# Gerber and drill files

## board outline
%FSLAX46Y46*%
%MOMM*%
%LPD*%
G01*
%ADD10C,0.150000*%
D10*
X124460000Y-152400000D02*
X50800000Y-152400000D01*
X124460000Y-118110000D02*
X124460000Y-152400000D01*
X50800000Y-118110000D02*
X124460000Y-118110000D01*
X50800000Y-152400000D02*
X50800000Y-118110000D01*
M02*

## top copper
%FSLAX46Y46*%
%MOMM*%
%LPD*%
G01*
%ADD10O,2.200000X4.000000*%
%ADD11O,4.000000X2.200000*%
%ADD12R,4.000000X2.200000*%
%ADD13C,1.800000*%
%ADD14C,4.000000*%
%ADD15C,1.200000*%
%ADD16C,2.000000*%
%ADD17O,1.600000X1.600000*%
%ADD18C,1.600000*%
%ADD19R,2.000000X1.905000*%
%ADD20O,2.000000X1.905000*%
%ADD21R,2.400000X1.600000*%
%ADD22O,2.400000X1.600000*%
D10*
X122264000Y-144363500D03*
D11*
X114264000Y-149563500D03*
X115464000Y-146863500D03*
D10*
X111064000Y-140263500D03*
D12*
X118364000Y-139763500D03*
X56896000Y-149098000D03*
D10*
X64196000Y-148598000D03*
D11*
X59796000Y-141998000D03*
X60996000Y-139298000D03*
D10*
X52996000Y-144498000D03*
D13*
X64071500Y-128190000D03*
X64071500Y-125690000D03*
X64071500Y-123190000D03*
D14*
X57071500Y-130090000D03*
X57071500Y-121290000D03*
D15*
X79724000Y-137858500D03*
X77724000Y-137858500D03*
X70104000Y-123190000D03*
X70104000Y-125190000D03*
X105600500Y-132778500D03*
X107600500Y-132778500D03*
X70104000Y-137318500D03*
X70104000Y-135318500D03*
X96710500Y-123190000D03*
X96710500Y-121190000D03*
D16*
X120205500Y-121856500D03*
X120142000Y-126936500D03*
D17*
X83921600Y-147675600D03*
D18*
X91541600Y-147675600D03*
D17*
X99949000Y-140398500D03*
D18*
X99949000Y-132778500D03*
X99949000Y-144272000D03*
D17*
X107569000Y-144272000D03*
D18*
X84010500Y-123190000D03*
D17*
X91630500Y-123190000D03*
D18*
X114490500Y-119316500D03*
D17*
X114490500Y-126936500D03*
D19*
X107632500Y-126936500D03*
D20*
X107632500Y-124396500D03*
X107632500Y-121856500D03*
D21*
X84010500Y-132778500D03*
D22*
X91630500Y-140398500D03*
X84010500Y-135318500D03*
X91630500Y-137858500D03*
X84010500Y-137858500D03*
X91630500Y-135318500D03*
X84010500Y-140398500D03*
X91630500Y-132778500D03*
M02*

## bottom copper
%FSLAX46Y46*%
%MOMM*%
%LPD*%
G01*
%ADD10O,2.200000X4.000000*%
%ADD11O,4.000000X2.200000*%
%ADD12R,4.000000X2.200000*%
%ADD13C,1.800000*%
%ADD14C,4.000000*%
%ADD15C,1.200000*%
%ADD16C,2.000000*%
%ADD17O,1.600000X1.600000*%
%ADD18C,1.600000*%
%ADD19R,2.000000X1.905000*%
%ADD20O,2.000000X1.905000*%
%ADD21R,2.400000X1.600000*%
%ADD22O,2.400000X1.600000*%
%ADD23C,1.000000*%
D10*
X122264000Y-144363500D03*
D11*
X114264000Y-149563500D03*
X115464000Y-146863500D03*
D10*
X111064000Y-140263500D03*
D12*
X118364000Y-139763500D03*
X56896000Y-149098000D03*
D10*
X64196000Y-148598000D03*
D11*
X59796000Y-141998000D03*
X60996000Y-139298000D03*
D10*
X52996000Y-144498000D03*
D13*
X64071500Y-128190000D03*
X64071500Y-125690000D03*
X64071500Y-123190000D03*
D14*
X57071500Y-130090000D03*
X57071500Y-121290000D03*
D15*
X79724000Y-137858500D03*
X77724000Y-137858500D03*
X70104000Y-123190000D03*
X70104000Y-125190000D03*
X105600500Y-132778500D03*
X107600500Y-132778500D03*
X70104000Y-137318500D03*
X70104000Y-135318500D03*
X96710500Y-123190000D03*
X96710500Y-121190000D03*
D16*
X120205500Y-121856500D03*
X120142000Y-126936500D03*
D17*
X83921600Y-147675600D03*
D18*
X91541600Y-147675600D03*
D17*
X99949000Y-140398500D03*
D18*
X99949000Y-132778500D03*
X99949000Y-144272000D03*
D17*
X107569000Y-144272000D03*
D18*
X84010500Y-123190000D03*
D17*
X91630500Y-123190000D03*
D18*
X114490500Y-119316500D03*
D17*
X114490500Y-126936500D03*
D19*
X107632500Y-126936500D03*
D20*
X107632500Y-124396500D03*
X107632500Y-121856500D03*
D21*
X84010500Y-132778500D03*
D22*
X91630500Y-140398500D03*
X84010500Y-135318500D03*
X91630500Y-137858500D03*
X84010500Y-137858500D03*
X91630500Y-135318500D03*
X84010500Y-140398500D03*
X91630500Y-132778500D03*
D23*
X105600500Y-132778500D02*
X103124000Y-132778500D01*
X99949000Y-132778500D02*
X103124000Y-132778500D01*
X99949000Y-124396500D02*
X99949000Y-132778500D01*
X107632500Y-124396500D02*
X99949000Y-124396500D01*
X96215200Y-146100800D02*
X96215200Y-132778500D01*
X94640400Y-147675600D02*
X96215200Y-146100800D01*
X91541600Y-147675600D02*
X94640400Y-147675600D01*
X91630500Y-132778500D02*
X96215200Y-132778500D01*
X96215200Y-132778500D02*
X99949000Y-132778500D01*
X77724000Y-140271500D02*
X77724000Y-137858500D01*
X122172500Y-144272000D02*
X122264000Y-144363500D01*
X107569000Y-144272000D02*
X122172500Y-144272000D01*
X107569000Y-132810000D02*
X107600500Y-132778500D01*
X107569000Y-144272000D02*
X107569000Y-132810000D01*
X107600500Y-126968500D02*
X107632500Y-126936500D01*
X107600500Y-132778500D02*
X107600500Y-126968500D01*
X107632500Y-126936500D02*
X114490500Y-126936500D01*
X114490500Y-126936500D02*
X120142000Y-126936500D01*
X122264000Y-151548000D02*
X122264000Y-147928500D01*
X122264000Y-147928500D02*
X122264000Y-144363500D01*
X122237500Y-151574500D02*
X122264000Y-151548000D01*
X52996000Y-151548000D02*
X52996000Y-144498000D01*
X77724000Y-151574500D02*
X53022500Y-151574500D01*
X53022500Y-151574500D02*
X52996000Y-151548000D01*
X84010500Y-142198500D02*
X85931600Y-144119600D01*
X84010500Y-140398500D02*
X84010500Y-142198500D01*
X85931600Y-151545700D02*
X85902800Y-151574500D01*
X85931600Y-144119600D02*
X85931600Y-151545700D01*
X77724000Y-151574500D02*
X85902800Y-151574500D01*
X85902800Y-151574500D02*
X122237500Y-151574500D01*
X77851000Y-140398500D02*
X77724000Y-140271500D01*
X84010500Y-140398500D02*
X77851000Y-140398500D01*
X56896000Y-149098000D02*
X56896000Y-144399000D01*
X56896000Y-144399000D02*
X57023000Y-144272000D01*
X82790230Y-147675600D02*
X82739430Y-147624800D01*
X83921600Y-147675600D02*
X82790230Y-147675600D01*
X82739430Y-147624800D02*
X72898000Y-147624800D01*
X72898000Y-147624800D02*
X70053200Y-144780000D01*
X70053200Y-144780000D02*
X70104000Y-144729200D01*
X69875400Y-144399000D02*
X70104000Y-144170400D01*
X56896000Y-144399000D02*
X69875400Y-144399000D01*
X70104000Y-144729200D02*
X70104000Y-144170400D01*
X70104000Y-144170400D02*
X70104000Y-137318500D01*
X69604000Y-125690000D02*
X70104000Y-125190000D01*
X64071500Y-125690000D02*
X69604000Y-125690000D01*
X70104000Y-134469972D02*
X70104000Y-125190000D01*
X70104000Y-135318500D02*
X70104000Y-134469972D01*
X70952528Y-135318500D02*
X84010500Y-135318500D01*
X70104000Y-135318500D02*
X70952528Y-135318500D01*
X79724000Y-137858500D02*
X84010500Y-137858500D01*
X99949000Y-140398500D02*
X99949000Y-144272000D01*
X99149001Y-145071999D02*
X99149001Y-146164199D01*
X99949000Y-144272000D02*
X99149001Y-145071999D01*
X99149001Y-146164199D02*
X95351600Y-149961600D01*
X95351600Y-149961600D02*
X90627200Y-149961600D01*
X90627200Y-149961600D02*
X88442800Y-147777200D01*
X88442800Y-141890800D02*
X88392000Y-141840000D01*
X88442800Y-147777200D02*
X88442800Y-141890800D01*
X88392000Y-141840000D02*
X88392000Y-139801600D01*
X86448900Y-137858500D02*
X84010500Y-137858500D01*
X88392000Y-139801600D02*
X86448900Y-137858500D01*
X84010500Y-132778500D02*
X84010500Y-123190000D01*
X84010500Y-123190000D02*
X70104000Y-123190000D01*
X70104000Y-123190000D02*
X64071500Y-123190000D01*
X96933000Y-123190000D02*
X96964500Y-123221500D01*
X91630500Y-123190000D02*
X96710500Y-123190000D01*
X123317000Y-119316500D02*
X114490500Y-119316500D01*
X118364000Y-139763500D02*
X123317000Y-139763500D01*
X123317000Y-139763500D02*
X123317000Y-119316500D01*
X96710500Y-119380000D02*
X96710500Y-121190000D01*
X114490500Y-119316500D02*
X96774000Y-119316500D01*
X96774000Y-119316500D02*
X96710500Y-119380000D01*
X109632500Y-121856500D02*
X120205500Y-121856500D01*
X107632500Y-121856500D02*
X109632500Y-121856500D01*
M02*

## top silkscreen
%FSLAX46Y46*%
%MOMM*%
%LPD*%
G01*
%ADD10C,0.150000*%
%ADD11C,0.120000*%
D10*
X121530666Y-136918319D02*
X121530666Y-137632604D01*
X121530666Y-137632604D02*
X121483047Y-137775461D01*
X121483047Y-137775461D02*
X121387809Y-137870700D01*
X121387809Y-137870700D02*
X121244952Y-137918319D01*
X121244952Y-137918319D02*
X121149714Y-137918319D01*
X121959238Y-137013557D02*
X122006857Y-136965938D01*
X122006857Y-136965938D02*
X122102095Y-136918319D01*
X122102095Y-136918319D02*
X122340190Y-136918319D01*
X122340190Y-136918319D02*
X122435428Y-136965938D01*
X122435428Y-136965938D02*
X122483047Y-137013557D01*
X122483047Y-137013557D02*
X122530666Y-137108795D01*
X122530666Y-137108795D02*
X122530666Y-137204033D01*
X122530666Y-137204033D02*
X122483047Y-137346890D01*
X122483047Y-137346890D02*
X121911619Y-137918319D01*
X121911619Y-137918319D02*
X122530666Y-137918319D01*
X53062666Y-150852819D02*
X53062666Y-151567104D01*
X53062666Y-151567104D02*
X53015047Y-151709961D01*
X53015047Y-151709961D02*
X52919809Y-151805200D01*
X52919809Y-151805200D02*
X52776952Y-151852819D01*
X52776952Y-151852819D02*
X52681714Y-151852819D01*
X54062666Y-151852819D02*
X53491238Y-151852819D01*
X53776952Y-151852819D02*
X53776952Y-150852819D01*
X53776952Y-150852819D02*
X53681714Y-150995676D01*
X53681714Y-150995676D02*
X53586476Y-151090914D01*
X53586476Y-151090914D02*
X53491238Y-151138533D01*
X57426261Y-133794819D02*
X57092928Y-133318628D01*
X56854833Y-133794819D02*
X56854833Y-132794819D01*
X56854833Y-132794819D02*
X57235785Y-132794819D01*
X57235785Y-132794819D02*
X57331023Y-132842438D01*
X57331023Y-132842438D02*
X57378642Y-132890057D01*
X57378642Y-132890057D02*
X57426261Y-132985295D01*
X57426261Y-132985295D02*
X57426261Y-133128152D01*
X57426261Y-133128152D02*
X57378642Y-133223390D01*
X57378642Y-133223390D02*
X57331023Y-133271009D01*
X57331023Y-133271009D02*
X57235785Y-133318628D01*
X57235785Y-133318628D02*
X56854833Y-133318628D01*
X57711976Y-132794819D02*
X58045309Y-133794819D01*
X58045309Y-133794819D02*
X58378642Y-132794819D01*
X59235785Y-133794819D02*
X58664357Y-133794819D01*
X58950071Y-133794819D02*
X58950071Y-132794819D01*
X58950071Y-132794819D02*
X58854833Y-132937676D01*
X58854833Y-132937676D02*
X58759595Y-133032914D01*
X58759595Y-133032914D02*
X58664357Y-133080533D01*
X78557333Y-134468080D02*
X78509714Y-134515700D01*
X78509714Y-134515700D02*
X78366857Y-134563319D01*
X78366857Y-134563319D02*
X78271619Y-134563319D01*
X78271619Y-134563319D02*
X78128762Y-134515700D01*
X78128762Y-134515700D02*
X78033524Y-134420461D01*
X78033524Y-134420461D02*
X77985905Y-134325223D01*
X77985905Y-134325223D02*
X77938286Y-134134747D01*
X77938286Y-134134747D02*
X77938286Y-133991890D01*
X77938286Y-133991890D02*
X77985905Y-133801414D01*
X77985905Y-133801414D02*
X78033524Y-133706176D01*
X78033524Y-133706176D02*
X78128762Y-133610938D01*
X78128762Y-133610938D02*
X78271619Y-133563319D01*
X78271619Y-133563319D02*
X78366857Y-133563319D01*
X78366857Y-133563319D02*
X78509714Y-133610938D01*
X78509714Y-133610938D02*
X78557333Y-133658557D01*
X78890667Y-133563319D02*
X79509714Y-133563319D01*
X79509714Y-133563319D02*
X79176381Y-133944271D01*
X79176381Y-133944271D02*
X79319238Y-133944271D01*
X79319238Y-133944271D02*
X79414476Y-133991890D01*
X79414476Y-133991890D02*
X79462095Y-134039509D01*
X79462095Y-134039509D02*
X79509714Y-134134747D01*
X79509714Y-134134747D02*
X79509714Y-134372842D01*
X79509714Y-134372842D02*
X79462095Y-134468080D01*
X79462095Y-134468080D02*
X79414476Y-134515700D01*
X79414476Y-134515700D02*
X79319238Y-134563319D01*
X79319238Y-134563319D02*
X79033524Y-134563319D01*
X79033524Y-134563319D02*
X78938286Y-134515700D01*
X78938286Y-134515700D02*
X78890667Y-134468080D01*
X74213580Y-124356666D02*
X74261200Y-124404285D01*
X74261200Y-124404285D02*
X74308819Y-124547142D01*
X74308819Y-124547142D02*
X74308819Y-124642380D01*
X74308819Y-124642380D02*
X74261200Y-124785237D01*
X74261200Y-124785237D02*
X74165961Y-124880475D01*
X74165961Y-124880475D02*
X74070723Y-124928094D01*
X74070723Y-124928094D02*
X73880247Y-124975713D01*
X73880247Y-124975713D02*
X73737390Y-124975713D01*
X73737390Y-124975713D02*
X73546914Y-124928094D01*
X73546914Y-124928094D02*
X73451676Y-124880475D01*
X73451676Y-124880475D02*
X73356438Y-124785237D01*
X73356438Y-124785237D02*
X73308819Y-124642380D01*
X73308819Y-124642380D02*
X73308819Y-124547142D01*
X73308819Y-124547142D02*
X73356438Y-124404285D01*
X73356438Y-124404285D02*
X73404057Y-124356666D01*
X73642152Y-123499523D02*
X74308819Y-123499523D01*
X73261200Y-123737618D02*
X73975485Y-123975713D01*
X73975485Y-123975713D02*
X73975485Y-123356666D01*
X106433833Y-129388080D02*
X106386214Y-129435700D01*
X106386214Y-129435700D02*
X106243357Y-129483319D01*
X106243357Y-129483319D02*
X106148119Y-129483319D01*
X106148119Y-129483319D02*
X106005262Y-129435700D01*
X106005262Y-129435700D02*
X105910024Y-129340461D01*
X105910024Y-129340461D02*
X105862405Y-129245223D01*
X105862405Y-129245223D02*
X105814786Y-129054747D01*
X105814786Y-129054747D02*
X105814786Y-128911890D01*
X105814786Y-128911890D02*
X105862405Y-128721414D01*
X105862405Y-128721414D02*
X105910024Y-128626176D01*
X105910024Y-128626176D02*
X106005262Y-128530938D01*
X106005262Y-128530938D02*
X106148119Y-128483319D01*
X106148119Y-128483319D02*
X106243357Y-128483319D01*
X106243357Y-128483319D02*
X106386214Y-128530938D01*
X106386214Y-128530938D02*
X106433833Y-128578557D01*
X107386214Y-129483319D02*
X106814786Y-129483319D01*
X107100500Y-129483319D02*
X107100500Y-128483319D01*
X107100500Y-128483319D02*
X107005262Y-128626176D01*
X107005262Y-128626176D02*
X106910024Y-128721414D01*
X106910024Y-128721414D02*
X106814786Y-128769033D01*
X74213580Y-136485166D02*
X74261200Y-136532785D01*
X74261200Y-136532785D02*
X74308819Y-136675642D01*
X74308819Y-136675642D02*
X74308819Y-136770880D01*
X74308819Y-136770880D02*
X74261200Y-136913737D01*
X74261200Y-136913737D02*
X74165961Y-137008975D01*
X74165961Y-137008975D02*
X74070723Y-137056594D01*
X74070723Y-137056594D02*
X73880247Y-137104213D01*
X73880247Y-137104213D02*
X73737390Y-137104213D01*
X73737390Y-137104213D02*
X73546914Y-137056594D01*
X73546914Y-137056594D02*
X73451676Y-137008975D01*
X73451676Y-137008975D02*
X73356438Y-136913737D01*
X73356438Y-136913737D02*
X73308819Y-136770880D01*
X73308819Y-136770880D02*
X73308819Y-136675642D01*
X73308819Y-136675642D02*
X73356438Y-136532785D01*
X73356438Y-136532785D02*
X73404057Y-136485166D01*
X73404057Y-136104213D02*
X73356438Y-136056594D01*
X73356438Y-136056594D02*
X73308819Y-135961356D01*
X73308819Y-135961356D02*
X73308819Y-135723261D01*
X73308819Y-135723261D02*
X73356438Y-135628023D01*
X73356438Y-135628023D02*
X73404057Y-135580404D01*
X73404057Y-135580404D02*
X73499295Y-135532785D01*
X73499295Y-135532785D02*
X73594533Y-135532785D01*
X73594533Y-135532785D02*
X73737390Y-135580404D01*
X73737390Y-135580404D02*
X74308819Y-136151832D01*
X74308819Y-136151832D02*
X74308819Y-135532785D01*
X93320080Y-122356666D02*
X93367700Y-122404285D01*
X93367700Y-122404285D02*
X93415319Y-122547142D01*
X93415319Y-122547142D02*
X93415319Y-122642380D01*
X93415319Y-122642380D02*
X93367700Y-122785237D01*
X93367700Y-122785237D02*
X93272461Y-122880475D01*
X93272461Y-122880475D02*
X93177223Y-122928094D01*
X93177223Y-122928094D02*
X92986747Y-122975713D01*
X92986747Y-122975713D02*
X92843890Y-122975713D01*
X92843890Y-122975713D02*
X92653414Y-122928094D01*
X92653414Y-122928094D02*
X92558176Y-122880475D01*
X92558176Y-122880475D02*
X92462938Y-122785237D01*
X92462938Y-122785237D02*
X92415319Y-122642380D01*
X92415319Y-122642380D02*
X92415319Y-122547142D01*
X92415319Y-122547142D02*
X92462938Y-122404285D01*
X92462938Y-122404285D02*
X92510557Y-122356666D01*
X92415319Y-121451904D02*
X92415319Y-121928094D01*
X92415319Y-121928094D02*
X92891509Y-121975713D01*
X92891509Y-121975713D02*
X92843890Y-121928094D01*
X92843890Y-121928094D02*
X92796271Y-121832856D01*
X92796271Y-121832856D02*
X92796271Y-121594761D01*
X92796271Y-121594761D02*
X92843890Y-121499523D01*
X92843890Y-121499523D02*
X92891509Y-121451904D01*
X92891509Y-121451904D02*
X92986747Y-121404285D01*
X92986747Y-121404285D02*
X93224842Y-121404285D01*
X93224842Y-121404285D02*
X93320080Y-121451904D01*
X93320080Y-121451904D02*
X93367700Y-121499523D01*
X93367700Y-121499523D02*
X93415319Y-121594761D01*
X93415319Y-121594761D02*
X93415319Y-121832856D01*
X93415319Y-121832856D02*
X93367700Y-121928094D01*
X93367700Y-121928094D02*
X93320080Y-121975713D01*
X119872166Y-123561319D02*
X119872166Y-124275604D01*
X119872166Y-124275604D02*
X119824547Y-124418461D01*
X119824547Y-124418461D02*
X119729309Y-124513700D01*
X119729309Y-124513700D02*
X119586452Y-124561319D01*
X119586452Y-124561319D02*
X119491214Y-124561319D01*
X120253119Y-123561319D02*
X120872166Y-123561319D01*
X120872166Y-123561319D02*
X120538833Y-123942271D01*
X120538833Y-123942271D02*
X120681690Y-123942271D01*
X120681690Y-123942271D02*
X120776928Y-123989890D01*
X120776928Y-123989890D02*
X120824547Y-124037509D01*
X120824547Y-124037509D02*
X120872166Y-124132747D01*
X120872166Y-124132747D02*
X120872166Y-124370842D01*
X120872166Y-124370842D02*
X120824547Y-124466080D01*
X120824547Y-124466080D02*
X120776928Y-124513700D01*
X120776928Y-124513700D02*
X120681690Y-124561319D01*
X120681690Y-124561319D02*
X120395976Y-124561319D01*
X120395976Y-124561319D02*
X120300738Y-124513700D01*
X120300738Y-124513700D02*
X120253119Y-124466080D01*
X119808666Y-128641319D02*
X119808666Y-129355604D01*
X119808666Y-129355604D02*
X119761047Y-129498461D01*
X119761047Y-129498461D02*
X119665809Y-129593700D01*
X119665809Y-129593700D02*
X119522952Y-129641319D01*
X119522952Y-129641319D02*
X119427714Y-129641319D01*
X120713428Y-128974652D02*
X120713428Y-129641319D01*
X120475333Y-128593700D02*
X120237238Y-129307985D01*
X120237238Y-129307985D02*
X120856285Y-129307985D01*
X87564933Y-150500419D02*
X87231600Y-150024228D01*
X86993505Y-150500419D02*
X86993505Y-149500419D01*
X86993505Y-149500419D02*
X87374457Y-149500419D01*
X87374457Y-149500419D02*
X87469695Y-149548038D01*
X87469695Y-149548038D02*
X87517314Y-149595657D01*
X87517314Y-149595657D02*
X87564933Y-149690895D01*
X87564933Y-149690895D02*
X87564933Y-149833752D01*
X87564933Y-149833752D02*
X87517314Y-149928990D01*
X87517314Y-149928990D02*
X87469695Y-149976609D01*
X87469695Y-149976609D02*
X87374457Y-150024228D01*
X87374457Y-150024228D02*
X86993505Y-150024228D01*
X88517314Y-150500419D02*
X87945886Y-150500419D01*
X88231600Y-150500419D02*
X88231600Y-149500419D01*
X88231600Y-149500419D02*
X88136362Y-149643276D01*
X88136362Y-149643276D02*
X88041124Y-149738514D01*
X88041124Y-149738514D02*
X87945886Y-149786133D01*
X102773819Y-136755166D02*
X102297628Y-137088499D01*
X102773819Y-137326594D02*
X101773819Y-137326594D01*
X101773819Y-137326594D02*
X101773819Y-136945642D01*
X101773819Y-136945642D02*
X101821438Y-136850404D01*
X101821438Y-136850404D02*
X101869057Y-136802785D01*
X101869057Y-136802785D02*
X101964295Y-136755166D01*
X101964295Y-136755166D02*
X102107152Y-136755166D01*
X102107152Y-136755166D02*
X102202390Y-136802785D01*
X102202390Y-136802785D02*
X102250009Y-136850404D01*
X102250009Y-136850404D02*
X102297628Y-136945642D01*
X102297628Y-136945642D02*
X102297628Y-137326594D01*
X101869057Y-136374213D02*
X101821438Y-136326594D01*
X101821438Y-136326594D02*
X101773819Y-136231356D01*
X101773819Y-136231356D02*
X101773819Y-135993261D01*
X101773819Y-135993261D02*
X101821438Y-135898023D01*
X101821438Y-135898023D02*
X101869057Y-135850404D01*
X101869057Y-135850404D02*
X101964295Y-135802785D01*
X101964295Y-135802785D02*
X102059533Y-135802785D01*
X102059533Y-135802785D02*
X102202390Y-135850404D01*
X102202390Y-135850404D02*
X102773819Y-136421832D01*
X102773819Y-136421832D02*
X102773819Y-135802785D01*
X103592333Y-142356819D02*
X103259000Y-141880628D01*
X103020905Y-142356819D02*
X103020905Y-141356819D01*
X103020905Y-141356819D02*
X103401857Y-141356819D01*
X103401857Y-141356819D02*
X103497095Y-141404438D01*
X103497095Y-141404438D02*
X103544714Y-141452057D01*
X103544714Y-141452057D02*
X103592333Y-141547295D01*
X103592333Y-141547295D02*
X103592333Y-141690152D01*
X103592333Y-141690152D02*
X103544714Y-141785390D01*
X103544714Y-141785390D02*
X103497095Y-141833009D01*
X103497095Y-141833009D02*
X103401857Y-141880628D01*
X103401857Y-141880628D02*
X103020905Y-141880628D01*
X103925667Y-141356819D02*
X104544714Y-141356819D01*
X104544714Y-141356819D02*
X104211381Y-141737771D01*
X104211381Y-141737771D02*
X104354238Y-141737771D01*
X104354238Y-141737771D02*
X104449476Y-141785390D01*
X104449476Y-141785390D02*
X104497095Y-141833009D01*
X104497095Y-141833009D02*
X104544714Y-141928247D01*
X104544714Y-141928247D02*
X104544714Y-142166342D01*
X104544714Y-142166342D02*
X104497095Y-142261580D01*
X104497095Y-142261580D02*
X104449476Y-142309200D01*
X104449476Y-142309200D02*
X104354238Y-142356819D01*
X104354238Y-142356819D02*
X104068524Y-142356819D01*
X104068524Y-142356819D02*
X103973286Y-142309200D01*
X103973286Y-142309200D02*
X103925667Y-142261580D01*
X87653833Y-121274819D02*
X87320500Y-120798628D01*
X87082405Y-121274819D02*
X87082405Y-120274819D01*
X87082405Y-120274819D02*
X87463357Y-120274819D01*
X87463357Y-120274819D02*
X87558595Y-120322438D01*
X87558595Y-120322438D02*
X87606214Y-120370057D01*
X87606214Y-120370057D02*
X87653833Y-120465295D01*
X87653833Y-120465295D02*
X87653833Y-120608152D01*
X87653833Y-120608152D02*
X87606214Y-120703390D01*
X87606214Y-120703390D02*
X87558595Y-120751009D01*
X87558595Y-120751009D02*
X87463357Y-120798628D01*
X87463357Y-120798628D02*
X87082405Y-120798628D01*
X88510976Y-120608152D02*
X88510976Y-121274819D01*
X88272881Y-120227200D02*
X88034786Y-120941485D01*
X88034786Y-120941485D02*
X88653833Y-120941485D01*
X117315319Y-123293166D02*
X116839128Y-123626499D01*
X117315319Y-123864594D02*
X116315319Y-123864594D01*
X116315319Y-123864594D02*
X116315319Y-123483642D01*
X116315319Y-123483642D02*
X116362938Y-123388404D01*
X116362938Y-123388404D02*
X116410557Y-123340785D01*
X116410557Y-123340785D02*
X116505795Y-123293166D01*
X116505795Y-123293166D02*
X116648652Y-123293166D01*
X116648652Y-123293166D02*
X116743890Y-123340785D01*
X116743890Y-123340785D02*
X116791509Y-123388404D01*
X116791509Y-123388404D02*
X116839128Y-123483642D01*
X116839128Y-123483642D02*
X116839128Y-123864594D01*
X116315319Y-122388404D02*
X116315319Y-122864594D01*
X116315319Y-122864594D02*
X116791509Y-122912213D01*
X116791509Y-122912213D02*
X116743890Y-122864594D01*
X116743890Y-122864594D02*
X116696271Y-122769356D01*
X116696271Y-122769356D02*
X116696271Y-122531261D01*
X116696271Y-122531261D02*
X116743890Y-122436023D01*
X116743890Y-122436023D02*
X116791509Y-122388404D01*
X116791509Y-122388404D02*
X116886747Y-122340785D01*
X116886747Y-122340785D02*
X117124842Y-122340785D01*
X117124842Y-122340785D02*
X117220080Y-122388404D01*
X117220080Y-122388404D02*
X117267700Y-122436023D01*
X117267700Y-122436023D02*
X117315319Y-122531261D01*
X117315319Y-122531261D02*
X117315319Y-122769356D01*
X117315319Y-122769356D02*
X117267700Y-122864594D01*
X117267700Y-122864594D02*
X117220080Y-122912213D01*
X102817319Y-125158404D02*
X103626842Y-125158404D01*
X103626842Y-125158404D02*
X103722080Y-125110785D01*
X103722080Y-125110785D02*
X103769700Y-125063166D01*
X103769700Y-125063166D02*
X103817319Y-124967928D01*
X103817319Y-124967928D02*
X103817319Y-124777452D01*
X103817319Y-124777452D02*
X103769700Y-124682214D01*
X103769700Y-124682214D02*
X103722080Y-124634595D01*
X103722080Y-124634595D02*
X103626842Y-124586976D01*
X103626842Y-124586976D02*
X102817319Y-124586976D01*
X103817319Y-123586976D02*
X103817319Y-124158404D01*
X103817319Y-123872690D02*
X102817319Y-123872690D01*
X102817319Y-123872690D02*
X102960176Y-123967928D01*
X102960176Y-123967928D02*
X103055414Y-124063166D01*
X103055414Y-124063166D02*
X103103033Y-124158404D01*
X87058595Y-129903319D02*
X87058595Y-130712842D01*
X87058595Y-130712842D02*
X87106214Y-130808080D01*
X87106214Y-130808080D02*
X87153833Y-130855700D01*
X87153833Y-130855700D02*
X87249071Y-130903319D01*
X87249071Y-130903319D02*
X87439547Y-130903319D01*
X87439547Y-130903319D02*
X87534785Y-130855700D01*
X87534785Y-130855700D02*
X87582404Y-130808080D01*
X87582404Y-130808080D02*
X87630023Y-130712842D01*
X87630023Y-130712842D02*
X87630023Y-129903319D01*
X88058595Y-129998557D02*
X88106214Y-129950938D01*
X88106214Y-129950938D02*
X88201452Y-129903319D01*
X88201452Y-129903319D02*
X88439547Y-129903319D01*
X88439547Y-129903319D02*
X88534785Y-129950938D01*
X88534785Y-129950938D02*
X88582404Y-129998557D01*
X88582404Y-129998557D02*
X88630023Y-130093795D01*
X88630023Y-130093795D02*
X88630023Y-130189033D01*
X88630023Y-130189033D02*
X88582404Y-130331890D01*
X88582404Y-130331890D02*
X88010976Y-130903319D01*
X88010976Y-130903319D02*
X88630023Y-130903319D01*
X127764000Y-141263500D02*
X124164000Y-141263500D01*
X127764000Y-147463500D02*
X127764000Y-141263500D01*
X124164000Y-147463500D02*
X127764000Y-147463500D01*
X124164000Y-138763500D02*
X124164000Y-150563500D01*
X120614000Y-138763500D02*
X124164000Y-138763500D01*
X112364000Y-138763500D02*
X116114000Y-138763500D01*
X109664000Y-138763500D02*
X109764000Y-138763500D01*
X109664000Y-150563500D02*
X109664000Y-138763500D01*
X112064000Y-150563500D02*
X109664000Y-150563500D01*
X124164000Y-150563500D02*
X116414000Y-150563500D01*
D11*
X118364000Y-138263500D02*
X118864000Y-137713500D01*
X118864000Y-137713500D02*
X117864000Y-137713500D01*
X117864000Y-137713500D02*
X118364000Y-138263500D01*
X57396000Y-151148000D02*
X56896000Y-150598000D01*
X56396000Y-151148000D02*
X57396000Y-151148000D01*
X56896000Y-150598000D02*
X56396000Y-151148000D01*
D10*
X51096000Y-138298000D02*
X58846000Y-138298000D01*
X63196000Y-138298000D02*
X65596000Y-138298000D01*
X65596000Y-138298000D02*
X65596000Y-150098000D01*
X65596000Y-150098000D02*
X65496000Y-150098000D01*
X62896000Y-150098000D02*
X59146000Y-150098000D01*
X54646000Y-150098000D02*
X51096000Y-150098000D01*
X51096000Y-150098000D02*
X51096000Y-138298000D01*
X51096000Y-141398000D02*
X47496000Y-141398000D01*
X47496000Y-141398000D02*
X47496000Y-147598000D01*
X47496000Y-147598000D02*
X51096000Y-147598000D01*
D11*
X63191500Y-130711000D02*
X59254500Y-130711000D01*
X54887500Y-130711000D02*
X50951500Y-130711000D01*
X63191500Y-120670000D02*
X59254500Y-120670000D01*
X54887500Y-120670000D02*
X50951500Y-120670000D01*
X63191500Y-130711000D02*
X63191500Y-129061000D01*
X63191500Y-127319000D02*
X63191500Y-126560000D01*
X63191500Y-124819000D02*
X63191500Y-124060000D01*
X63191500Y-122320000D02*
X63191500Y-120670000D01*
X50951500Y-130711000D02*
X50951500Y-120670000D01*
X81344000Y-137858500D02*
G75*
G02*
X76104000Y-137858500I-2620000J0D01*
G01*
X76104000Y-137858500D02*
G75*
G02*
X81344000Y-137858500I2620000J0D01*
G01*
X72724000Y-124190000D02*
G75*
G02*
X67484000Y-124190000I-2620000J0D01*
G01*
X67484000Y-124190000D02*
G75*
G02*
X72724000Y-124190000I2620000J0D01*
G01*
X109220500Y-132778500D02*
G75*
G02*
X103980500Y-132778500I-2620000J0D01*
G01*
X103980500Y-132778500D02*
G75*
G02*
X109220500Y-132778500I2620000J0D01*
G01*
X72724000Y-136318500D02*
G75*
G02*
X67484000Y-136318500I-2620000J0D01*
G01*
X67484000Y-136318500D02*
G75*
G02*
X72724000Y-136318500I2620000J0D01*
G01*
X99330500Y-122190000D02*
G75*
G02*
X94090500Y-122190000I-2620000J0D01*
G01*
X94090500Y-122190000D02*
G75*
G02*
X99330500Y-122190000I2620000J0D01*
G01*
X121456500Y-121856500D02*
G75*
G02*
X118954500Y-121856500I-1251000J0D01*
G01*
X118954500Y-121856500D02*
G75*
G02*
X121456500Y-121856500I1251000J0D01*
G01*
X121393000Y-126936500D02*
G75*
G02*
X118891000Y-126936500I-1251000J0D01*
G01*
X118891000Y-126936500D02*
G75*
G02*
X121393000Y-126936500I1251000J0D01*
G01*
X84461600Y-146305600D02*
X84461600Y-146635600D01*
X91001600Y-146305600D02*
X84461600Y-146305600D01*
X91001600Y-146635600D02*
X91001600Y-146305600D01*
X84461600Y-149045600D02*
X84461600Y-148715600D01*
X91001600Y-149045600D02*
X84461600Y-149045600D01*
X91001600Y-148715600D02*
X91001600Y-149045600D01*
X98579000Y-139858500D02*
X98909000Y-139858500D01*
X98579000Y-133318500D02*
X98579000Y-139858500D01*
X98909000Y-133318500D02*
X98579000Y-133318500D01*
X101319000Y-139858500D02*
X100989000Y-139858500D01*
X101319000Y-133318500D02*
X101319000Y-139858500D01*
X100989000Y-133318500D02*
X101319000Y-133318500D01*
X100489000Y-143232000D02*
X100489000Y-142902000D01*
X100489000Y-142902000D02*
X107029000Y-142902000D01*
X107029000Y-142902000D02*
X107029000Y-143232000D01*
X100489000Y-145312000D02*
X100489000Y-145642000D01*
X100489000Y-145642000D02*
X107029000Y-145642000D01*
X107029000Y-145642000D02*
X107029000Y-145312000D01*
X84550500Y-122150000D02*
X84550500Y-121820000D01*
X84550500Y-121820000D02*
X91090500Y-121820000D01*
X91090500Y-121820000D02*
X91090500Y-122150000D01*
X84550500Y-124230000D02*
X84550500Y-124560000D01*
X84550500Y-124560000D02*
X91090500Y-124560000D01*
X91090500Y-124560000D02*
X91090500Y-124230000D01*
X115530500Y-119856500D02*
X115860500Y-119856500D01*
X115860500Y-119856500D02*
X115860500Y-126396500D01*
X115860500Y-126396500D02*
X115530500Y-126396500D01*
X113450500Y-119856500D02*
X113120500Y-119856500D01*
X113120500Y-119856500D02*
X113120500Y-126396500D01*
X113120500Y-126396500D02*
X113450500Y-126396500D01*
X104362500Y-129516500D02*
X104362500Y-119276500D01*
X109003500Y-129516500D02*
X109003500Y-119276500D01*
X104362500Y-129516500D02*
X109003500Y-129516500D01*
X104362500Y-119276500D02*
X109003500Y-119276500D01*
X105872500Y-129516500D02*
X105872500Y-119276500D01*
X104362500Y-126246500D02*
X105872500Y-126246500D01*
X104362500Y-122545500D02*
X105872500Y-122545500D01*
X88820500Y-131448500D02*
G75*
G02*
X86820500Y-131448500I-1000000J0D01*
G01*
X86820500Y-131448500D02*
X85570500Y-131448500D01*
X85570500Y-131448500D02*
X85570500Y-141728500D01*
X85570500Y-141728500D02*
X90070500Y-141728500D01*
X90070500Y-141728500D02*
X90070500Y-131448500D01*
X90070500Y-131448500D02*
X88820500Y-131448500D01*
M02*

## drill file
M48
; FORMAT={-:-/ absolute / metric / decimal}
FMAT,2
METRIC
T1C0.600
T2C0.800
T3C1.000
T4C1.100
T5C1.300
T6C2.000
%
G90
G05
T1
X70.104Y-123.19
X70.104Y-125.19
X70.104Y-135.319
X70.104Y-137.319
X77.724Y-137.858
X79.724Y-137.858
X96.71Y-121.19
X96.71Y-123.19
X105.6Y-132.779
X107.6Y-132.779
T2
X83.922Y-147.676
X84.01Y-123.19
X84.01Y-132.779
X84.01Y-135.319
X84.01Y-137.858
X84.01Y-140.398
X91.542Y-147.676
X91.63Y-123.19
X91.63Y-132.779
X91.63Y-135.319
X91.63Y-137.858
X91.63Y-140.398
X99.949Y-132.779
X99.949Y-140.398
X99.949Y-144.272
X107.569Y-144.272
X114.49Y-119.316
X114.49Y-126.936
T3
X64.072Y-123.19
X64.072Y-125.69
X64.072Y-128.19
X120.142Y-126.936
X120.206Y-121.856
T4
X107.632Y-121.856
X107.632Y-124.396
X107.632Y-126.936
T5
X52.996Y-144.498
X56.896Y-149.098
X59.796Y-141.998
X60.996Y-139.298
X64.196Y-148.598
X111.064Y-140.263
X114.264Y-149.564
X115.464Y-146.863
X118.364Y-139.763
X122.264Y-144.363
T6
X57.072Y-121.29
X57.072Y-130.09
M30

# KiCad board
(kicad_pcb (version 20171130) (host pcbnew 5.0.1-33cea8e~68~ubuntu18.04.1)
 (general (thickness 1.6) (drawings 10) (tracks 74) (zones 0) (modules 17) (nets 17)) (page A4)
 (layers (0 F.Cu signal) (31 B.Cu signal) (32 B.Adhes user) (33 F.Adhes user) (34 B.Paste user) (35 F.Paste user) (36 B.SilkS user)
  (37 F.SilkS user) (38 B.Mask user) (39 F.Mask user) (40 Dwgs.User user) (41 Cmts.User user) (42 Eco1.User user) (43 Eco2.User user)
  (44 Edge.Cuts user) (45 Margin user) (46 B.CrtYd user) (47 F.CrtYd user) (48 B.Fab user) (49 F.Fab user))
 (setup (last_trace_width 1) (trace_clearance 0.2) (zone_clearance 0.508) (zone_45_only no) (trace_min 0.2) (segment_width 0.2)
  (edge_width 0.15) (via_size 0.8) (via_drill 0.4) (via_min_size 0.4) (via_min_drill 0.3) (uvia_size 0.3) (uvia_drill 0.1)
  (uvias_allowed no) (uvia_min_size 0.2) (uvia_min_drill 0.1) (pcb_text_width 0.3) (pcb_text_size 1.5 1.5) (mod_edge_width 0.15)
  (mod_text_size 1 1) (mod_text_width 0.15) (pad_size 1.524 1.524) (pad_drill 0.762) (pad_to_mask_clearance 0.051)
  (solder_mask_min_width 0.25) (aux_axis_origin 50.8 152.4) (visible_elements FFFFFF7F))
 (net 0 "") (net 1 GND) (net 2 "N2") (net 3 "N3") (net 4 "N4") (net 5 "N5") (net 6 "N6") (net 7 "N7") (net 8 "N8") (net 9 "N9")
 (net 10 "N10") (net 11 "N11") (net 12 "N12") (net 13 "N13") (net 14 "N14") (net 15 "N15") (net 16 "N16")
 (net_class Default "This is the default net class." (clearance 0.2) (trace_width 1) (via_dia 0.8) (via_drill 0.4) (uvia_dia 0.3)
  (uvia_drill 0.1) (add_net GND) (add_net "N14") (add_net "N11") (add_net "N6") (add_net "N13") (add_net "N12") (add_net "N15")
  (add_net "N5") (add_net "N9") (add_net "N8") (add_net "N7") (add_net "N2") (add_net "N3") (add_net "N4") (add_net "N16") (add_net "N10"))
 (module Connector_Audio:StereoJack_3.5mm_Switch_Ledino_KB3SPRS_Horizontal (layer F.Cu) (at 118.364 139.7635 180)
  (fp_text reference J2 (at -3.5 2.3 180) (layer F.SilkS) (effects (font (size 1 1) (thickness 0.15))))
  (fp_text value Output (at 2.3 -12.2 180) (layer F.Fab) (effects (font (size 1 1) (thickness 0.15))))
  (fp_line (start -9.4 -1.5) (end -5.8 -1.5) (layer F.SilkS) (width 0.15))
  (fp_line (start -9.4 -7.7) (end -9.4 -1.5) (layer F.SilkS) (width 0.15))
  (fp_line (start -5.8 -7.7) (end -9.4 -7.7) (layer F.SilkS) (width 0.15))
  (fp_line (start -5.8 1) (end -5.8 -10.8) (layer F.SilkS) (width 0.15))
  (fp_line (start -2.25 1) (end -5.8 1) (layer F.SilkS) (width 0.15))
  (fp_line (start 6 1) (end 2.25 1) (layer F.SilkS) (width 0.15))
  (fp_line (start 8.7 1) (end 8.6 1) (layer F.SilkS) (width 0.15))
  (fp_line (start 8.7 -10.8) (end 8.7 1) (layer F.SilkS) (width 0.15))
  (fp_line (start 6.3 -10.8) (end 8.7 -10.8) (layer F.SilkS) (width 0.15))
  (fp_line (start -5.8 -10.8) (end 1.95 -10.8) (layer F.SilkS) (width 0.15))
  (fp_line (start 0 1.5) (end -0.5 2.05) (layer F.SilkS) (width 0.12))
  (fp_line (start -0.5 2.05) (end 0.5 2.05) (layer F.SilkS) (width 0.12))
  (fp_line (start 0.5 2.05) (end 0 1.5) (layer F.SilkS) (width 0.12))
  (pad S thru_hole oval (at -3.9 -4.6 180) (size 2.2 4) (drill 1.3) (layers *.Cu *.Mask) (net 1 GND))
  (pad R thru_hole oval (at 4.1 -9.8 180) (size 4 2.2) (drill 1.3) (layers *.Cu *.Mask) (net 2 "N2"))
  (pad RN thru_hole oval (at 2.9 -7.1 180) (size 4 2.2) (drill 1.3) (layers *.Cu *.Mask) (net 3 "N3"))
  (pad TN thru_hole oval (at 7.3 -0.5 270) (size 4 2.2) (drill 1.3) (layers *.Cu *.Mask) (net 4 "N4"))
  (pad T thru_hole rect (at 0 0 180) (size 4 2.2) (drill 1.3) (layers *.Cu *.Mask) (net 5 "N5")))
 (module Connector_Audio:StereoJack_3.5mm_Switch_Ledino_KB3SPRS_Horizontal (layer F.Cu) (at 56.896 149.098)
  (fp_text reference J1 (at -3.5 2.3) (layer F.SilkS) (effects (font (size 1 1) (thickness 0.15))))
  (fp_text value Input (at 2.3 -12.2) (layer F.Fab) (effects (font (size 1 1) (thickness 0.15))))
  (fp_line (start 0.5 2.05) (end 0 1.5) (layer F.SilkS) (width 0.12))
  (fp_line (start -0.5 2.05) (end 0.5 2.05) (layer F.SilkS) (width 0.12))
  (fp_line (start 0 1.5) (end -0.5 2.05) (layer F.SilkS) (width 0.12))
  (fp_line (start -5.8 -10.8) (end 1.95 -10.8) (layer F.SilkS) (width 0.15))
  (fp_line (start 6.3 -10.8) (end 8.7 -10.8) (layer F.SilkS) (width 0.15))
  (fp_line (start 8.7 -10.8) (end 8.7 1) (layer F.SilkS) (width 0.15))
  (fp_line (start 8.7 1) (end 8.6 1) (layer F.SilkS) (width 0.15))
  (fp_line (start 6 1) (end 2.25 1) (layer F.SilkS) (width 0.15))
  (fp_line (start -2.25 1) (end -5.8 1) (layer F.SilkS) (width 0.15))
  (fp_line (start -5.8 1) (end -5.8 -10.8) (layer F.SilkS) (width 0.15))
  (fp_line (start -5.8 -7.7) (end -9.4 -7.7) (layer F.SilkS) (width 0.15))
  (fp_line (start -9.4 -7.7) (end -9.4 -1.5) (layer F.SilkS) (width 0.15))
  (fp_line (start -9.4 -1.5) (end -5.8 -1.5) (layer F.SilkS) (width 0.15))
  (pad T thru_hole rect (at 0 0) (size 4 2.2) (drill 1.3) (layers *.Cu *.Mask) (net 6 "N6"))
  (pad TN thru_hole oval (at 7.3 -0.5 90) (size 4 2.2) (drill 1.3) (layers *.Cu *.Mask) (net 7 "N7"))
  (pad RN thru_hole oval (at 2.9 -7.1) (size 4 2.2) (drill 1.3) (layers *.Cu *.Mask) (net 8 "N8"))
  (pad R thru_hole oval (at 4.1 -9.8) (size 4 2.2) (drill 1.3) (layers *.Cu *.Mask) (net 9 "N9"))
  (pad S thru_hole oval (at -3.9 -4.6) (size 2.2 4) (drill 1.3) (layers *.Cu *.Mask) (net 1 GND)))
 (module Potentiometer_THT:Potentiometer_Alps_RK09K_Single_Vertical (layer F.Cu) (at 64.0715 123.19 180)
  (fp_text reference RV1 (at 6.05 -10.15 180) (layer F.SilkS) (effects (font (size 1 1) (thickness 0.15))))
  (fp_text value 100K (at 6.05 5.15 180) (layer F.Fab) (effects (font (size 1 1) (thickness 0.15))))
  (fp_line (start 0.88 -7.521) (end 4.817 -7.521) (layer F.SilkS) (width 0.12))
  (fp_line (start 9.184 -7.521) (end 13.12 -7.521) (layer F.SilkS) (width 0.12))
  (fp_line (start 0.88 2.52) (end 4.817 2.52) (layer F.SilkS) (width 0.12))
  (fp_line (start 9.184 2.52) (end 13.12 2.52) (layer F.SilkS) (width 0.12))
  (fp_line (start 0.88 -7.521) (end 0.88 -5.871) (layer F.SilkS) (width 0.12))
  (fp_line (start 0.88 -4.129) (end 0.88 -3.37) (layer F.SilkS) (width 0.12))
  (fp_line (start 0.88 -1.629) (end 0.88 -0.87) (layer F.SilkS) (width 0.12))
  (fp_line (start 0.88 0.87) (end 0.88 2.52) (layer F.SilkS) (width 0.12))
  (fp_line (start 13.12 -7.521) (end 13.12 2.52) (layer F.SilkS) (width 0.12))
  (pad 3 thru_hole circle (at 0 -5 180) (size 1.8 1.8) (drill 1) (layers *.Cu *.Mask) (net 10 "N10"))
  (pad 2 thru_hole circle (at 0 -2.5 180) (size 1.8 1.8) (drill 1) (layers *.Cu *.Mask) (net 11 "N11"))
  (pad 1 thru_hole circle (at 0 0 180) (size 1.8 1.8) (drill 1) (layers *.Cu *.Mask) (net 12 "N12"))
  (pad "" np_thru_hole circle (at 7 -6.9 180) (size 4 4) (drill 2) (layers *.Cu *.Mask))
  (pad "" np_thru_hole circle (at 7 1.9 180) (size 4 4) (drill 2) (layers *.Cu *.Mask)))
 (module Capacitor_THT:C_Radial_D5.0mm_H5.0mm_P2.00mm (layer F.Cu) (at 77.724 137.8585)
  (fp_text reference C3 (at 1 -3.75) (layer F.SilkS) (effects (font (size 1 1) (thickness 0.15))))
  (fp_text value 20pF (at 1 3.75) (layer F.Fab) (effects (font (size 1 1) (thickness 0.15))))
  (fp_circle (center 1 0) (end 3.62 0) (layer F.SilkS) (width 0.12))
  (pad 2 thru_hole circle (at 2 0) (size 1.2 1.2) (drill 0.6) (layers *.Cu *.Mask) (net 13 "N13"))
  (pad 1 thru_hole circle (at 0 0) (size 1.2 1.2) (drill 0.6) (layers *.Cu *.Mask) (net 1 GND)))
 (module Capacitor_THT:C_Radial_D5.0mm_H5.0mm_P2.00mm (layer F.Cu) (at 70.104 123.19 270)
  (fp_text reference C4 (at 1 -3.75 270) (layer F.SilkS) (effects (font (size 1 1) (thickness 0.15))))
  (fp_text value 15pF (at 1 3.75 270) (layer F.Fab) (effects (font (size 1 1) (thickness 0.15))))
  (fp_circle (center 1 0) (end 3.62 0) (layer F.SilkS) (width 0.12))
  (pad 1 thru_hole circle (at 0 0 270) (size 1.2 1.2) (drill 0.6) (layers *.Cu *.Mask) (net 12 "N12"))
  (pad 2 thru_hole circle (at 2 0 270) (size 1.2 1.2) (drill 0.6) (layers *.Cu *.Mask) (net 11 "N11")))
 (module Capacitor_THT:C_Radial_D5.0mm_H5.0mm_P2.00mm (layer F.Cu) (at 105.6005 132.7785)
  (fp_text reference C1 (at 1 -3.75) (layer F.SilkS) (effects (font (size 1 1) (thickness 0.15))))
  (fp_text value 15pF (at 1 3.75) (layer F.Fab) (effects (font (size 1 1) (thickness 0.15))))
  (fp_circle (center 1 0) (end 3.62 0) (layer F.SilkS) (width 0.12))
  (pad 1 thru_hole circle (at 0 0) (size 1.2 1.2) (drill 0.6) (layers *.Cu *.Mask) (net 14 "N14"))
  (pad 2 thru_hole circle (at 2 0) (size 1.2 1.2) (drill 0.6) (layers *.Cu *.Mask) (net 1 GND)))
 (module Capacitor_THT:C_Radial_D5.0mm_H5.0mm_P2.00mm (layer F.Cu) (at 70.104 135.3185 270)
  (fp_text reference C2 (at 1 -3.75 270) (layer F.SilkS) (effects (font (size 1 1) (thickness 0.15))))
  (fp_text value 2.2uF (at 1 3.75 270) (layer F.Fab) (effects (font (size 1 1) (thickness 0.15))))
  (fp_circle (center 1 0) (end 3.62 0) (layer F.SilkS) (width 0.12))
  (pad 2 thru_hole circle (at 2 0 270) (size 1.2 1.2) (drill 0.6) (layers *.Cu *.Mask) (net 6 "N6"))
  (pad 1 thru_hole circle (at 0 0 270) (size 1.2 1.2) (drill 0.6) (layers *.Cu *.Mask) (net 11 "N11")))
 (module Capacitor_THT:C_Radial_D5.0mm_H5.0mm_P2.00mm (layer F.Cu) (at 96.7105 123.19 90)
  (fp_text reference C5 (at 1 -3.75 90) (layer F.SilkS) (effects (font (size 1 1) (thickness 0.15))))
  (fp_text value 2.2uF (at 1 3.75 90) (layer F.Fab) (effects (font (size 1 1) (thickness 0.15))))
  (fp_circle (center 1 0) (end 3.62 0) (layer F.SilkS) (width 0.12))
  (pad 1 thru_hole circle (at 0 0 90) (size 1.2 1.2) (drill 0.6) (layers *.Cu *.Mask) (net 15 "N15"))
  (pad 2 thru_hole circle (at 2 0 90) (size 1.2 1.2) (drill 0.6) (layers *.Cu *.Mask) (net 5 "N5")))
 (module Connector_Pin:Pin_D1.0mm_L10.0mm (layer F.Cu) (at 120.2055 121.8565)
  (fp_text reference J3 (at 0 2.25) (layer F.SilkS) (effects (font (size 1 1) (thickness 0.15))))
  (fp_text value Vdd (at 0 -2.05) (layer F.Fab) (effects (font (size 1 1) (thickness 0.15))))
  (fp_circle (center 0 0) (end 1.25 0.05) (layer F.SilkS) (width 0.12))
  (pad 1 thru_hole circle (at 0 0) (size 2 2) (drill 1) (layers *.Cu *.Mask) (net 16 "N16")))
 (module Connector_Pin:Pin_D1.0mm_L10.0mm (layer F.Cu) (at 120.142 126.9365)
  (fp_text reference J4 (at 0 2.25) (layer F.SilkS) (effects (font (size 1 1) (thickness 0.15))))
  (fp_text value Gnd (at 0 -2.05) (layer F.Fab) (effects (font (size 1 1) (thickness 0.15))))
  (fp_circle (center 0 0) (end 1.25 0.05) (layer F.SilkS) (width 0.12))
  (pad 1 thru_hole circle (at 0 0) (size 2 2) (drill 1) (layers *.Cu *.Mask) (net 1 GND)))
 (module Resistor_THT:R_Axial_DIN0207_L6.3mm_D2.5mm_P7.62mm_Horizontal (layer F.Cu) (at 91.5416 147.6756 180)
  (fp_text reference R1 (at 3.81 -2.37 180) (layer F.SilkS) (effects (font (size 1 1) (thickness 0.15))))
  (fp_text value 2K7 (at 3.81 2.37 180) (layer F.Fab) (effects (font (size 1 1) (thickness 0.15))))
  (fp_line (start 7.08 1.37) (end 7.08 1.04) (layer F.SilkS) (width 0.12))
  (fp_line (start 0.54 1.37) (end 7.08 1.37) (layer F.SilkS) (width 0.12))
  (fp_line (start 0.54 1.04) (end 0.54 1.37) (layer F.SilkS) (width 0.12))
  (fp_line (start 7.08 -1.37) (end 7.08 -1.04) (layer F.SilkS) (width 0.12))
  (fp_line (start 0.54 -1.37) (end 7.08 -1.37) (layer F.SilkS) (width 0.12))
  (fp_line (start 0.54 -1.04) (end 0.54 -1.37) (layer F.SilkS) (width 0.12))
  (pad 2 thru_hole oval (at 7.62 0 180) (size 1.6 1.6) (drill 0.8) (layers *.Cu *.Mask) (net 6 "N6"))
  (pad 1 thru_hole circle (at 0 0 180) (size 1.6 1.6) (drill 0.8) (layers *.Cu *.Mask) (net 14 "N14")))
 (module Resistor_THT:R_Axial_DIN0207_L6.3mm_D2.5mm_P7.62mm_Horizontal (layer F.Cu) (at 99.949 132.7785 270)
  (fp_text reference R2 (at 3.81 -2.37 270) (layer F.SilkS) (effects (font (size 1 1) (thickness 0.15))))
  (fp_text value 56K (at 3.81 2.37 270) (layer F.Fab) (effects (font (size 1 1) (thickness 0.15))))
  (fp_line (start 7.08 1.37) (end 7.08 1.04) (layer F.SilkS) (width 0.12))
  (fp_line (start 0.54 1.37) (end 7.08 1.37) (layer F.SilkS) (width 0.12))
  (fp_line (start 0.54 1.04) (end 0.54 1.37) (layer F.SilkS) (width 0.12))
  (fp_line (start 7.08 -1.37) (end 7.08 -1.04) (layer F.SilkS) (width 0.12))
  (fp_line (start 0.54 -1.37) (end 7.08 -1.37) (layer F.SilkS) (width 0.12))
  (fp_line (start 0.54 -1.04) (end 0.54 -1.37) (layer F.SilkS) (width 0.12))
  (pad 2 thru_hole oval (at 7.62 0 270) (size 1.6 1.6) (drill 0.8) (layers *.Cu *.Mask) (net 13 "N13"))
  (pad 1 thru_hole circle (at 0 0 270) (size 1.6 1.6) (drill 0.8) (layers *.Cu *.Mask) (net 14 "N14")))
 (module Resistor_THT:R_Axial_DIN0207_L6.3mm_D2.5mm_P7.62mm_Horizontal (layer F.Cu) (at 99.949 144.272)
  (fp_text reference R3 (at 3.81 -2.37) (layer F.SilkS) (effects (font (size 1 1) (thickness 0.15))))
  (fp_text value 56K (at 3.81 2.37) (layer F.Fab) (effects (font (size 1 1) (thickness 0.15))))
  (fp_line (start 0.54 -1.04) (end 0.54 -1.37) (layer F.SilkS) (width 0.12))
  (fp_line (start 0.54 -1.37) (end 7.08 -1.37) (layer F.SilkS) (width 0.12))
  (fp_line (start 7.08 -1.37) (end 7.08 -1.04) (layer F.SilkS) (width 0.12))
  (fp_line (start 0.54 1.04) (end 0.54 1.37) (layer F.SilkS) (width 0.12))
  (fp_line (start 0.54 1.37) (end 7.08 1.37) (layer F.SilkS) (width 0.12))
  (fp_line (start 7.08 1.37) (end 7.08 1.04) (layer F.SilkS) (width 0.12))
  (pad 1 thru_hole circle (at 0 0) (size 1.6 1.6) (drill 0.8) (layers *.Cu *.Mask) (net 13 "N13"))
  (pad 2 thru_hole oval (at 7.62 0) (size 1.6 1.6) (drill 0.8) (layers *.Cu *.Mask) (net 1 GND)))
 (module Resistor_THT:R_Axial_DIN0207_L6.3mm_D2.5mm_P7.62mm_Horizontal (layer F.Cu) (at 84.0105 123.19)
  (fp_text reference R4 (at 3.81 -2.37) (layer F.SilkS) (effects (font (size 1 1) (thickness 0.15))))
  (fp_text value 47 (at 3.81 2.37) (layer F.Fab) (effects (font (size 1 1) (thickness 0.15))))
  (fp_line (start 0.54 -1.04) (end 0.54 -1.37) (layer F.SilkS) (width 0.12))
  (fp_line (start 0.54 -1.37) (end 7.08 -1.37) (layer F.SilkS) (width 0.12))
  (fp_line (start 7.08 -1.37) (end 7.08 -1.04) (layer F.SilkS) (width 0.12))
  (fp_line (start 0.54 1.04) (end 0.54 1.37) (layer F.SilkS) (width 0.12))
  (fp_line (start 0.54 1.37) (end 7.08 1.37) (layer F.SilkS) (width 0.12))
  (fp_line (start 7.08 1.37) (end 7.08 1.04) (layer F.SilkS) (width 0.12))
  (pad 1 thru_hole circle (at 0 0) (size 1.6 1.6) (drill 0.8) (layers *.Cu *.Mask) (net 12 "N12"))
  (pad 2 thru_hole oval (at 7.62 0) (size 1.6 1.6) (drill 0.8) (layers *.Cu *.Mask) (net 15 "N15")))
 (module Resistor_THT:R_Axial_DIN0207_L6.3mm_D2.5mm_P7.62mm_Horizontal (layer F.Cu) (at 114.4905 119.3165 270)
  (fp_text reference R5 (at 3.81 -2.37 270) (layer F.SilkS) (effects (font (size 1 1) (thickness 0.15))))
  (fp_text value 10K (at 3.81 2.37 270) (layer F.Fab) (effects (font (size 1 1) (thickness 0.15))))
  (fp_line (start 0.54 -1.04) (end 0.54 -1.37) (layer F.SilkS) (width 0.12))
  (fp_line (start 0.54 -1.37) (end 7.08 -1.37) (layer F.SilkS) (width 0.12))
  (fp_line (start 7.08 -1.37) (end 7.08 -1.04) (layer F.SilkS) (width 0.12))
  (fp_line (start 0.54 1.04) (end 0.54 1.37) (layer F.SilkS) (width 0.12))
  (fp_line (start 0.54 1.37) (end 7.08 1.37) (layer F.SilkS) (width 0.12))
  (fp_line (start 7.08 1.37) (end 7.08 1.04) (layer F.SilkS) (width 0.12))
  (pad 1 thru_hole circle (at 0 0 270) (size 1.6 1.6) (drill 0.8) (layers *.Cu *.Mask) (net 5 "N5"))
  (pad 2 thru_hole oval (at 7.62 0 270) (size 1.6 1.6) (drill 0.8) (layers *.Cu *.Mask) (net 1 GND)))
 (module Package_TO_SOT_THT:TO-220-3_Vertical (layer F.Cu) (at 107.6325 126.9365 90)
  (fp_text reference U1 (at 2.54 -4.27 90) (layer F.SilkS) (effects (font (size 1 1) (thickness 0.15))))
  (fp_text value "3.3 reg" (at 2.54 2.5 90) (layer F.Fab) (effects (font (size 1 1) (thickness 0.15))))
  (fp_line (start -2.58 -3.27) (end 7.66 -3.27) (layer F.SilkS) (width 0.12))
  (fp_line (start -2.58 1.371) (end 7.66 1.371) (layer F.SilkS) (width 0.12))
  (fp_line (start -2.58 -3.27) (end -2.58 1.371) (layer F.SilkS) (width 0.12))
  (fp_line (start 7.66 -3.27) (end 7.66 1.371) (layer F.SilkS) (width 0.12))
  (fp_line (start -2.58 -1.76) (end 7.66 -1.76) (layer F.SilkS) (width 0.12))
  (fp_line (start 0.69 -3.27) (end 0.69 -1.76) (layer F.SilkS) (width 0.12))
  (fp_line (start 4.391 -3.27) (end 4.391 -1.76) (layer F.SilkS) (width 0.12))
  (pad 1 thru_hole rect (at 0 0 90) (size 1.905 2) (drill 1.1) (layers *.Cu *.Mask) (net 1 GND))
  (pad 2 thru_hole oval (at 2.54 0 90) (size 1.905 2) (drill 1.1) (layers *.Cu *.Mask) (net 14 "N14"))
  (pad 3 thru_hole oval (at 5.08 0 90) (size 1.905 2) (drill 1.1) (layers *.Cu *.Mask) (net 16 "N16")))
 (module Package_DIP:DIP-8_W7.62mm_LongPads (layer F.Cu) (at 84.0105 132.7785)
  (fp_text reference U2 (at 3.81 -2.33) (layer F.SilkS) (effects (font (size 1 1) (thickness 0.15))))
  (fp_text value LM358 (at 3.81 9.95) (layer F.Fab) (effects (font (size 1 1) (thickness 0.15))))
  (fp_arc (start 3.81 -1.33) (end 2.81 -1.33) (angle -180) (layer F.SilkS) (width 0.12))
  (fp_line (start 2.81 -1.33) (end 1.56 -1.33) (layer F.SilkS) (width 0.12))
  (fp_line (start 1.56 -1.33) (end 1.56 8.95) (layer F.SilkS) (width 0.12))
  (fp_line (start 1.56 8.95) (end 6.06 8.95) (layer F.SilkS) (width 0.12))
  (fp_line (start 6.06 8.95) (end 6.06 -1.33) (layer F.SilkS) (width 0.12))
  (fp_line (start 6.06 -1.33) (end 4.81 -1.33) (layer F.SilkS) (width 0.12))
  (pad 1 thru_hole rect (at 0 0) (size 2.4 1.6) (drill 0.8) (layers *.Cu *.Mask) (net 12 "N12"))
  (pad 5 thru_hole oval (at 7.62 7.62) (size 2.4 1.6) (drill 0.8) (layers *.Cu *.Mask))
  (pad 2 thru_hole oval (at 0 2.54) (size 2.4 1.6) (drill 0.8) (layers *.Cu *.Mask) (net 11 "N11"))
  (pad 6 thru_hole oval (at 7.62 5.08) (size 2.4 1.6) (drill 0.8) (layers *.Cu *.Mask))
  (pad 3 thru_hole oval (at 0 5.08) (size 2.4 1.6) (drill 0.8) (layers *.Cu *.Mask) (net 13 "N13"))
  (pad 7 thru_hole oval (at 7.62 2.54) (size 2.4 1.6) (drill 0.8) (layers *.Cu *.Mask))
  (pad 4 thru_hole oval (at 0 7.62) (size 2.4 1.6) (drill 0.8) (layers *.Cu *.Mask) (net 1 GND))
  (pad 8 thru_hole oval (at 7.62 0) (size 2.4 1.6) (drill 0.8) (layers *.Cu *.Mask) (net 14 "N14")))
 (gr_line (start 124.46 152.4) (end 50.8 152.4) (layer Edge.Cuts) (width 0.15))
 (gr_line (start 124.46 118.11) (end 124.46 152.4) (layer Edge.Cuts) (width 0.15))
 (gr_line (start 50.8 118.11) (end 124.46 118.11) (layer Edge.Cuts) (width 0.15))
 (gr_line (start 50.8 152.4) (end 50.8 118.11) (layer Edge.Cuts) (width 0.15))
 (segment (start 105.6005 132.7785) (end 103.124 132.7785) (width 1) (layer B.Cu) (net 14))
 (segment (start 99.949 132.7785) (end 103.124 132.7785) (width 1) (layer B.Cu) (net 14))
 (segment (start 99.949 124.3965) (end 99.949 132.7785) (width 1) (layer B.Cu) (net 14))
 (segment (start 107.6325 124.3965) (end 99.949 124.3965) (width 1) (layer B.Cu) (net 14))
 (segment (start 96.2152 146.1008) (end 96.2152 132.7785) (width 1) (layer B.Cu) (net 14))
 (segment (start 94.6404 147.6756) (end 96.2152 146.1008) (width 1) (layer B.Cu) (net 14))
 (segment (start 91.5416 147.6756) (end 94.6404 147.6756) (width 1) (layer B.Cu) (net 14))
 (segment (start 91.6305 132.7785) (end 96.2152 132.7785) (width 1) (layer B.Cu) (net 14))
 (segment (start 96.2152 132.7785) (end 99.949 132.7785) (width 1) (layer B.Cu) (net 14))
 (segment (start 77.724 140.2715) (end 77.724 137.8585) (width 1) (layer B.Cu) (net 1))
 (segment (start 122.1725 144.272) (end 122.264 144.3635) (width 1) (layer B.Cu) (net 1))
 (segment (start 107.569 144.272) (end 122.1725 144.272) (width 1) (layer B.Cu) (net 1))
 (segment (start 107.569 132.81) (end 107.6005 132.7785) (width 1) (layer B.Cu) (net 1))
 (segment (start 107.569 144.272) (end 107.569 132.81) (width 1) (layer B.Cu) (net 1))
 (segment (start 107.6005 126.9685) (end 107.6325 126.9365) (width 1) (layer B.Cu) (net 1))
 (segment (start 107.6005 132.7785) (end 107.6005 126.9685) (width 1) (layer B.Cu) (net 1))
 (segment (start 107.6325 126.9365) (end 114.4905 126.9365) (width 1) (layer B.Cu) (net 1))
 (segment (start 114.4905 126.9365) (end 120.142 126.9365) (width 1) (layer B.Cu) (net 1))
 (segment (start 122.264 151.548) (end 122.264 147.9285) (width 1) (layer B.Cu) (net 1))
 (segment (start 122.264 147.9285) (end 122.264 144.3635) (width 1) (layer B.Cu) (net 1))
 (segment (start 122.2375 151.5745) (end 122.264 151.548) (width 1) (layer B.Cu) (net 1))
 (segment (start 52.996 151.548) (end 52.996 144.498) (width 1) (layer B.Cu) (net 1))
 (segment (start 77.724 151.5745) (end 53.0225 151.5745) (width 1) (layer B.Cu) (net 1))
 (segment (start 53.0225 151.5745) (end 52.996 151.548) (width 1) (layer B.Cu) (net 1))
 (segment (start 84.0105 142.1985) (end 85.9316 144.1196) (width 1) (layer B.Cu) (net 1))
 (segment (start 84.0105 140.3985) (end 84.0105 142.1985) (width 1) (layer B.Cu) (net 1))
 (segment (start 85.9316 151.5457) (end 85.9028 151.5745) (width 1) (layer B.Cu) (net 1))
 (segment (start 85.9316 144.1196) (end 85.9316 151.5457) (width 1) (layer B.Cu) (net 1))
 (segment (start 77.724 151.5745) (end 85.9028 151.5745) (width 1) (layer B.Cu) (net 1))
 (segment (start 85.9028 151.5745) (end 122.2375 151.5745) (width 1) (layer B.Cu) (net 1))
 (segment (start 77.851 140.3985) (end 77.724 140.2715) (width 1) (layer B.Cu) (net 1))
 (segment (start 84.0105 140.3985) (end 77.851 140.3985) (width 1) (layer B.Cu) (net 1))
 (segment (start 56.896 149.098) (end 56.896 144.399) (width 1) (layer B.Cu) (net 6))
 (segment (start 56.896 144.399) (end 57.023 144.272) (width 1) (layer B.Cu) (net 6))
 (segment (start 82.79023 147.6756) (end 82.73943 147.6248) (width 1) (layer B.Cu) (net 6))
 (segment (start 83.9216 147.6756) (end 82.79023 147.6756) (width 1) (layer B.Cu) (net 6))
 (segment (start 82.73943 147.6248) (end 72.898 147.6248) (width 1) (layer B.Cu) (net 6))
 (segment (start 72.898 147.6248) (end 70.0532 144.78) (width 1) (layer B.Cu) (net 6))
 (segment (start 70.0532 144.78) (end 70.104 144.7292) (width 1) (layer B.Cu) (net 6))
 (segment (start 69.8754 144.399) (end 70.104 144.1704) (width 1) (layer B.Cu) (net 6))
 (segment (start 56.896 144.399) (end 69.8754 144.399) (width 1) (layer B.Cu) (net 6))
 (segment (start 70.104 144.7292) (end 70.104 144.1704) (width 1) (layer B.Cu) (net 6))
 (segment (start 70.104 144.1704) (end 70.104 137.3185) (width 1) (layer B.Cu) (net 6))
 (segment (start 69.604 125.69) (end 70.104 125.19) (width 1) (layer B.Cu) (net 11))
 (segment (start 64.0715 125.69) (end 69.604 125.69) (width 1) (layer B.Cu) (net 11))
 (segment (start 70.104 134.469972) (end 70.104 125.19) (width 1) (layer B.Cu) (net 11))
 (segment (start 70.104 135.3185) (end 70.104 134.469972) (width 1) (layer B.Cu) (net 11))
 (segment (start 70.952528 135.3185) (end 84.0105 135.3185) (width 1) (layer B.Cu) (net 11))
 (segment (start 70.104 135.3185) (end 70.952528 135.3185) (width 1) (layer B.Cu) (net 11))
 (segment (start 79.724 137.8585) (end 84.0105 137.8585) (width 1) (layer B.Cu) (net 13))
 (segment (start 99.949 140.3985) (end 99.949 144.272) (width 1) (layer B.Cu) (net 13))
 (segment (start 99.149001 145.071999) (end 99.149001 146.164199) (width 1) (layer B.Cu) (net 13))
 (segment (start 99.949 144.272) (end 99.149001 145.071999) (width 1) (layer B.Cu) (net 13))
 (segment (start 99.149001 146.164199) (end 95.3516 149.9616) (width 1) (layer B.Cu) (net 13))
 (segment (start 95.3516 149.9616) (end 90.6272 149.9616) (width 1) (layer B.Cu) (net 13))
 (segment (start 90.6272 149.9616) (end 88.4428 147.7772) (width 1) (layer B.Cu) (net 13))
 (segment (start 88.4428 141.8908) (end 88.392 141.84) (width 1) (layer B.Cu) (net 13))
 (segment (start 88.4428 147.7772) (end 88.4428 141.8908) (width 1) (layer B.Cu) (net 13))
 (segment (start 88.392 141.84) (end 88.392 139.8016) (width 1) (layer B.Cu) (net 13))
 (segment (start 86.4489 137.8585) (end 84.0105 137.8585) (width 1) (layer B.Cu) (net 13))
 (segment (start 88.392 139.8016) (end 86.4489 137.8585) (width 1) (layer B.Cu) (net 13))
 (segment (start 84.0105 132.7785) (end 84.0105 123.19) (width 1) (layer B.Cu) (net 12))
 (segment (start 84.0105 123.19) (end 70.104 123.19) (width 1) (layer B.Cu) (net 12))
 (segment (start 70.104 123.19) (end 64.0715 123.19) (width 1) (layer B.Cu) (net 12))
 (segment (start 96.933 123.19) (end 96.9645 123.2215) (width 1) (layer B.Cu) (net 15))
 (segment (start 91.6305 123.19) (end 96.7105 123.19) (width 1) (layer B.Cu) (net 15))
 (segment (start 123.317 119.3165) (end 114.4905 119.3165) (width 1) (layer B.Cu) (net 5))
 (segment (start 118.364 139.7635) (end 123.317 139.7635) (width 1) (layer B.Cu) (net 5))
 (segment (start 123.317 139.7635) (end 123.317 119.3165) (width 1) (layer B.Cu) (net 5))
 (segment (start 96.7105 119.38) (end 96.7105 121.19) (width 1) (layer B.Cu) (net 5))
 (segment (start 114.4905 119.3165) (end 96.774 119.3165) (width 1) (layer B.Cu) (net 5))
 (segment (start 96.774 119.3165) (end 96.7105 119.38) (width 1) (layer B.Cu) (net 5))
 (segment (start 109.6325 121.8565) (end 120.2055 121.8565) (width 1) (layer B.Cu) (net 16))
 (segment (start 107.6325 121.8565) (end 109.6325 121.8565) (width 1) (layer B.Cu) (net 16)))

